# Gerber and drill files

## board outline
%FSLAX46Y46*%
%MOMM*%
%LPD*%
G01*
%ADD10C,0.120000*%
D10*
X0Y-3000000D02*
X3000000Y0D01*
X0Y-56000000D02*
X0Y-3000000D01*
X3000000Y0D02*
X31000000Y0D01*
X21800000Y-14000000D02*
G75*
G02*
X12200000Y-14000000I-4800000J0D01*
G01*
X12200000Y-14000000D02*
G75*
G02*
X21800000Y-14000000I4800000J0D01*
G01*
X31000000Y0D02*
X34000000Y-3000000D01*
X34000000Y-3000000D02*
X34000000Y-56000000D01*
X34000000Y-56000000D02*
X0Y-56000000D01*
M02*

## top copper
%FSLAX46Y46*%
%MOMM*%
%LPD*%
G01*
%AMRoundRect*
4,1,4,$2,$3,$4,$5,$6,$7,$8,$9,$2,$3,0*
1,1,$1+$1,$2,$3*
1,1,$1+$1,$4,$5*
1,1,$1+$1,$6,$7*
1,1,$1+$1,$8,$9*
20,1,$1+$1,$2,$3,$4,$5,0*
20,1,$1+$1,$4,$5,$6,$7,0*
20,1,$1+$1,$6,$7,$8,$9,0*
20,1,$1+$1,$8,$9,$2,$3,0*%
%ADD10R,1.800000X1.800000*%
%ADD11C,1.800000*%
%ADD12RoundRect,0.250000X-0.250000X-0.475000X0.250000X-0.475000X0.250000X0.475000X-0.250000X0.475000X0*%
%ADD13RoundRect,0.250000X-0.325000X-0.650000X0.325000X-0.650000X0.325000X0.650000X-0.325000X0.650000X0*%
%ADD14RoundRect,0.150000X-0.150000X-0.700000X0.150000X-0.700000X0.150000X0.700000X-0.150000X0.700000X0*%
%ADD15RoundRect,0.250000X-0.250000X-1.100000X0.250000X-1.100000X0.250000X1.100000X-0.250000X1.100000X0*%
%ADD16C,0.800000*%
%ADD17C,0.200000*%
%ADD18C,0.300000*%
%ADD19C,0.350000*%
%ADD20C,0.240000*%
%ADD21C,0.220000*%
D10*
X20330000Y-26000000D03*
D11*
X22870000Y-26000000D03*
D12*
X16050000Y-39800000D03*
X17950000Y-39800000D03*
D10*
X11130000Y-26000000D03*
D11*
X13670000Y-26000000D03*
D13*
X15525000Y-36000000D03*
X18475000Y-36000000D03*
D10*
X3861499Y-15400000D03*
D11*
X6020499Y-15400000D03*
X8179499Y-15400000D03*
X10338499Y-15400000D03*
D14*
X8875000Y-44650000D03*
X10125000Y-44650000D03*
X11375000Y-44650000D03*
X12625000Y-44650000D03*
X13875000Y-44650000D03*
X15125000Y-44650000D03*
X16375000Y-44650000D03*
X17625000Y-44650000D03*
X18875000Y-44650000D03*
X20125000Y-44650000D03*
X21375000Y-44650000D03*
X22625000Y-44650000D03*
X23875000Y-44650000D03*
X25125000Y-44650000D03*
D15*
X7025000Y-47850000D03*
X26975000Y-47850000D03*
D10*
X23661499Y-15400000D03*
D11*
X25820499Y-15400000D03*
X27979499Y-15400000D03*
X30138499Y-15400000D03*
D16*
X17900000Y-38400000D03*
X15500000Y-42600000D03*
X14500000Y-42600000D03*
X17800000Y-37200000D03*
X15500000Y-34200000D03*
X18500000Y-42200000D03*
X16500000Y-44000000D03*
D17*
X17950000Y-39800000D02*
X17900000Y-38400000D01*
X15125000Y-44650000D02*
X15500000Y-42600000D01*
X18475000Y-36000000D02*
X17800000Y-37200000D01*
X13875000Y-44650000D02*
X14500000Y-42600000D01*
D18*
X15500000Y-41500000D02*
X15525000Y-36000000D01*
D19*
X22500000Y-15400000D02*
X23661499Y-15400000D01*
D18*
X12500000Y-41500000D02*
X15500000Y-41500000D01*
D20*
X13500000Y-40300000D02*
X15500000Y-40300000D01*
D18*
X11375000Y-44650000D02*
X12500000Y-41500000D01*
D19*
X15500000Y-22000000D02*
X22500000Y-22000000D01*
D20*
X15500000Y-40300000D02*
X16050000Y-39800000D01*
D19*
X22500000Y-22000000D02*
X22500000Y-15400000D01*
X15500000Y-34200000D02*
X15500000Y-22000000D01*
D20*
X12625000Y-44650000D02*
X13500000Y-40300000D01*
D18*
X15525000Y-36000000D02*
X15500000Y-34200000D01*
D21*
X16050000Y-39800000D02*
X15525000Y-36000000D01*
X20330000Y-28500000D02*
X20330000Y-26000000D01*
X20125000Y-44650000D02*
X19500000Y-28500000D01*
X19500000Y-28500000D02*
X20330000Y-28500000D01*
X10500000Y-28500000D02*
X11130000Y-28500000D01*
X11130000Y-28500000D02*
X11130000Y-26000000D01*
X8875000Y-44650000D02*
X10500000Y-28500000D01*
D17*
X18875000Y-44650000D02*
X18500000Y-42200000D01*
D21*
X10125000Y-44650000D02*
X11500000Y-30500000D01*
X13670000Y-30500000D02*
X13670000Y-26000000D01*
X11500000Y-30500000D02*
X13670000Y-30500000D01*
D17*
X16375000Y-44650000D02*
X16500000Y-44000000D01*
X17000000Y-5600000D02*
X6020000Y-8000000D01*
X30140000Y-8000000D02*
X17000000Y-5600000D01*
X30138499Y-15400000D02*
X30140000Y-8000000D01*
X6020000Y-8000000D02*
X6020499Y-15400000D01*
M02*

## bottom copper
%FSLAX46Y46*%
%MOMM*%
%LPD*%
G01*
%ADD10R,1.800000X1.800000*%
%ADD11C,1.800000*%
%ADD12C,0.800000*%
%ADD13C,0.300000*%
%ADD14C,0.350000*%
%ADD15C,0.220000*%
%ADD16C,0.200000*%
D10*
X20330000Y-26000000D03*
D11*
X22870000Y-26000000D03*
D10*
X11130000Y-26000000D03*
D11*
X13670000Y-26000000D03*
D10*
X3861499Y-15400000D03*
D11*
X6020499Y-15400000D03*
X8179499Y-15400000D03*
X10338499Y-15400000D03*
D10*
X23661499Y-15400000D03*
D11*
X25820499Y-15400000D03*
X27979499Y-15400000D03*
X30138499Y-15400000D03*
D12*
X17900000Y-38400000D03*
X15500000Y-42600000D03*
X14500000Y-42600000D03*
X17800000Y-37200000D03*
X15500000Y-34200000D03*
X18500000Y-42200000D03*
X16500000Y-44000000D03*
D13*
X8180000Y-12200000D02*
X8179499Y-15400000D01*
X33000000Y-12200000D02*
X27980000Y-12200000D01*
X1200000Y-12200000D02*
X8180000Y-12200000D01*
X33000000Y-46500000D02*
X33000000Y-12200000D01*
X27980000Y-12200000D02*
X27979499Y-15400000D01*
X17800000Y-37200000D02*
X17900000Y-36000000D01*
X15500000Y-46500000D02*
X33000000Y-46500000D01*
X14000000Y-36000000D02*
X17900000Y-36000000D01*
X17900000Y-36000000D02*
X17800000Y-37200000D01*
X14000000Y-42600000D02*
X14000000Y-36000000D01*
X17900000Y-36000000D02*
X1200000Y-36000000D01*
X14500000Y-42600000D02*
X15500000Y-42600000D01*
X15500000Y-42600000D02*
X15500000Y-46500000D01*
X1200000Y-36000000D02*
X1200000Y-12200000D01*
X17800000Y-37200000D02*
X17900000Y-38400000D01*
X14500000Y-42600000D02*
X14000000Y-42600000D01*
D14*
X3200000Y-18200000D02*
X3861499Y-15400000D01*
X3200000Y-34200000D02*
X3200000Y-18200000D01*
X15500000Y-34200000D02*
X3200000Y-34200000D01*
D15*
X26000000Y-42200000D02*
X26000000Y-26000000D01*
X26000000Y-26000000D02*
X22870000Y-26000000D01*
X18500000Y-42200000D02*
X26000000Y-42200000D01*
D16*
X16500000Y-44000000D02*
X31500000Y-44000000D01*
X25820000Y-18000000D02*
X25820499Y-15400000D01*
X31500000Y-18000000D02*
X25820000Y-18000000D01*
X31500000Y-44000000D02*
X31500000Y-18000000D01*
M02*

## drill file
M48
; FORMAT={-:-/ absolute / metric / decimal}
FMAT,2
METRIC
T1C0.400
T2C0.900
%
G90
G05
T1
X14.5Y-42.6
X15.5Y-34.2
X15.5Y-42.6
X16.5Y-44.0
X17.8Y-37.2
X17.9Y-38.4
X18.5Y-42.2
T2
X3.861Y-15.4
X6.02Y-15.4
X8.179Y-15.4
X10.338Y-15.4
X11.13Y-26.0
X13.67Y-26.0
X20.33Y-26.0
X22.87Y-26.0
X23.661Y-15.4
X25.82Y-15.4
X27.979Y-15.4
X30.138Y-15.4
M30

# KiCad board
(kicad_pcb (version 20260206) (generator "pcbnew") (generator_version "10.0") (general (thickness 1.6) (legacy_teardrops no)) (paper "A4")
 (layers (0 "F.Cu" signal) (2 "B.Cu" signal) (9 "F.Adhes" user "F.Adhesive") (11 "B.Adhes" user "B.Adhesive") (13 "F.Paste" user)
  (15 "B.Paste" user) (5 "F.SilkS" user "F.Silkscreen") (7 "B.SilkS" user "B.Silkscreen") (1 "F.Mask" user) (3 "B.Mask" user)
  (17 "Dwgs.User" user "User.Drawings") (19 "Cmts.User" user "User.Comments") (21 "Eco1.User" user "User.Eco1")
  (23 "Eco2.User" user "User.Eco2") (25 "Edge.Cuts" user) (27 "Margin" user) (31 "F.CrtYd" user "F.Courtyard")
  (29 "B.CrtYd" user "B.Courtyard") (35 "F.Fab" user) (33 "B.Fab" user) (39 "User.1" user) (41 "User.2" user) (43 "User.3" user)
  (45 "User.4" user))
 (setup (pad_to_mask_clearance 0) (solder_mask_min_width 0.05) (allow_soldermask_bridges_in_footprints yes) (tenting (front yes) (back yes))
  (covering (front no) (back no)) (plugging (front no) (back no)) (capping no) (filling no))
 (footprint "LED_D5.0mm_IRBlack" (layer "F.Cu") (at 20.33 26)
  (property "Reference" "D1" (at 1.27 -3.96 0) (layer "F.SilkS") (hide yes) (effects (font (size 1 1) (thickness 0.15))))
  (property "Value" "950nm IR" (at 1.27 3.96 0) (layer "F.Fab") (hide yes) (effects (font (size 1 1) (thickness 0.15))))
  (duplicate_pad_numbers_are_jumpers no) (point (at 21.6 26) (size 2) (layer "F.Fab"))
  (pad "1" thru_hole rect (at 0 0) (size 1.8 1.8) (drill 0.9) (layers "*.Cu" "*.Mask") (remove_unused_layers no) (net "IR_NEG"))
  (pad "2" thru_hole circle (at 2.54 0) (size 1.8 1.8) (drill 0.9) (layers "*.Cu" "*.Mask") (remove_unused_layers no) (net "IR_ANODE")))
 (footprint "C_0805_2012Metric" (layer "F.Cu") (at 17 39.8)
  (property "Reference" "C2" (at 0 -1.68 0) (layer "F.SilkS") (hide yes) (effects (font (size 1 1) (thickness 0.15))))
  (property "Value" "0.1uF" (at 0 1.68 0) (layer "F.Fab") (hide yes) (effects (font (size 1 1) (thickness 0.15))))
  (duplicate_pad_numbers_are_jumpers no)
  (pad "1" smd roundrect (at -0.95 0) (size 1 1.45) (layers "F.Cu" "F.Mask" "F.Paste") (roundrect_rratio 0.25) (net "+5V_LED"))
  (pad "2" smd roundrect (at 0.95 0) (size 1 1.45) (layers "F.Cu" "F.Mask" "F.Paste") (roundrect_rratio 0.25) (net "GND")))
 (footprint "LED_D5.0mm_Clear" (layer "F.Cu") (at 11.13 26)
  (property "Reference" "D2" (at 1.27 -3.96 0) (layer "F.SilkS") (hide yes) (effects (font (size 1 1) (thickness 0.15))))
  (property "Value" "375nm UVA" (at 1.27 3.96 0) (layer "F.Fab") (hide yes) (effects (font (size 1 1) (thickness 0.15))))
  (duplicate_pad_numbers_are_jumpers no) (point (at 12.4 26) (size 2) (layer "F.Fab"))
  (pad "1" thru_hole rect (at 0 0) (size 1.8 1.8) (drill 0.9) (layers "*.Cu" "*.Mask") (remove_unused_layers no) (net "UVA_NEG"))
  (pad "2" thru_hole circle (at 2.54 0) (size 1.8 1.8) (drill 0.9) (layers "*.Cu" "*.Mask") (remove_unused_layers no) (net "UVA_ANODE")))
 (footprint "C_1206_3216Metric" (layer "F.Cu") (at 17 36)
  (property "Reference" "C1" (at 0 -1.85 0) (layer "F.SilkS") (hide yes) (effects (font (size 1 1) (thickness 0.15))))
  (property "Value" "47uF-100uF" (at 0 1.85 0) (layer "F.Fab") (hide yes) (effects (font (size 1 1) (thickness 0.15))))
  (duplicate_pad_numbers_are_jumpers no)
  (pad "1" smd roundrect (at -1.475 0) (size 1.15 1.8) (layers "F.Cu" "F.Mask" "F.Paste") (roundrect_rratio 0.217391) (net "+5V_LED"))
  (pad "2" smd roundrect (at 1.475 0) (size 1.15 1.8) (layers "F.Cu" "F.Mask" "F.Paste") (roundrect_rratio 0.217391) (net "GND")))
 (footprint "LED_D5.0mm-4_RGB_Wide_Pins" (layer "F.Cu") (at 3.861499 15.4)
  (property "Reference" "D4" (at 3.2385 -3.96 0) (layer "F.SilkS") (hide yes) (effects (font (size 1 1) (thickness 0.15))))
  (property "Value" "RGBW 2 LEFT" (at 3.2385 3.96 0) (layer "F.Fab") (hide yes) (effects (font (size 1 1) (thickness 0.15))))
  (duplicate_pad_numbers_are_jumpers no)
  (pad "1" thru_hole rect (at 0 0) (size 1.8 1.8) (drill 0.9) (layers "*.Cu" "*.Mask") (remove_unused_layers no) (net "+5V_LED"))
  (pad "2" thru_hole circle (at 2.159 0) (size 1.8 1.8) (drill 0.9) (layers "*.Cu" "*.Mask") (remove_unused_layers no) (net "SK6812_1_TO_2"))
  (pad "3" thru_hole circle (at 4.318 0) (size 1.8 1.8) (drill 0.9) (layers "*.Cu" "*.Mask") (remove_unused_layers no) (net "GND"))
  (pad "4" thru_hole circle (at 6.477 0) (size 1.8 1.8) (drill 0.9) (layers "*.Cu" "*.Mask") (remove_unused_layers no)))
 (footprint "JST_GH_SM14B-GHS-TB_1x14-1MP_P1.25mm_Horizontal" (layer "F.Cu") (at 17 46.5)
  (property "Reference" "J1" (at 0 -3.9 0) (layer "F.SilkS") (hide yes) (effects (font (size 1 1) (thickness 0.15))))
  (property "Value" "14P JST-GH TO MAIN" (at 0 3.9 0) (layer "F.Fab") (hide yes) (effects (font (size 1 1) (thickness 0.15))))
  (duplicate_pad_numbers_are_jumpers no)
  (pad "1" smd roundrect (at -8.125 -1.85) (size 0.6 1.7) (layers "F.Cu" "F.Mask" "F.Paste") (roundrect_rratio 0.25) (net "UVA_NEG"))
  (pad "2" smd roundrect (at -6.875 -1.85) (size 0.6 1.7) (layers "F.Cu" "F.Mask" "F.Paste") (roundrect_rratio 0.25) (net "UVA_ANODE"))
  (pad "3" smd roundrect (at -5.625 -1.85) (size 0.6 1.7) (layers "F.Cu" "F.Mask" "F.Paste") (roundrect_rratio 0.25) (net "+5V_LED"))
  (pad "4" smd roundrect (at -4.375 -1.85) (size 0.6 1.7) (layers "F.Cu" "F.Mask" "F.Paste") (roundrect_rratio 0.25) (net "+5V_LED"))
  (pad "5" smd roundrect (at -3.125 -1.85) (size 0.6 1.7) (layers "F.Cu" "F.Mask" "F.Paste") (roundrect_rratio 0.25) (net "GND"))
  (pad "6" smd roundrect (at -1.875 -1.85) (size 0.6 1.7) (layers "F.Cu" "F.Mask" "F.Paste") (roundrect_rratio 0.25) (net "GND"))
  (pad "7" smd roundrect (at -0.625 -1.85) (size 0.6 1.7) (layers "F.Cu" "F.Mask" "F.Paste") (roundrect_rratio 0.25) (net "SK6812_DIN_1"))
  (pad "8" smd roundrect (at 0.625 -1.85) (size 0.6 1.7) (layers "F.Cu" "F.Mask" "F.Paste") (roundrect_rratio 0.25))
  (pad "9" smd roundrect (at 1.875 -1.85) (size 0.6 1.7) (layers "F.Cu" "F.Mask" "F.Paste") (roundrect_rratio 0.25) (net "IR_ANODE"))
  (pad "10" smd roundrect (at 3.125 -1.85) (size 0.6 1.7) (layers "F.Cu" "F.Mask" "F.Paste") (roundrect_rratio 0.25) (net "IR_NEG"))
  (pad "11" smd roundrect (at 4.375 -1.85) (size 0.6 1.7) (layers "F.Cu" "F.Mask" "F.Paste") (roundrect_rratio 0.25))
  (pad "12" smd roundrect (at 5.625 -1.85) (size 0.6 1.7) (layers "F.Cu" "F.Mask" "F.Paste") (roundrect_rratio 0.25))
  (pad "13" smd roundrect (at 6.875 -1.85) (size 0.6 1.7) (layers "F.Cu" "F.Mask" "F.Paste") (roundrect_rratio 0.25))
  (pad "14" smd roundrect (at 8.125 -1.85) (size 0.6 1.7) (layers "F.Cu" "F.Mask" "F.Paste") (roundrect_rratio 0.25))
  (pad "MP" smd roundrect (at -9.975 1.35) (size 1 2.7) (layers "F.Cu" "F.Mask" "F.Paste") (roundrect_rratio 0.25))
  (pad "MP" smd roundrect (at 9.975 1.35) (size 1 2.7) (layers "F.Cu" "F.Mask" "F.Paste") (roundrect_rratio 0.25)))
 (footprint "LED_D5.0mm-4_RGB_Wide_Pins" (layer "F.Cu") (at 23.661499 15.4)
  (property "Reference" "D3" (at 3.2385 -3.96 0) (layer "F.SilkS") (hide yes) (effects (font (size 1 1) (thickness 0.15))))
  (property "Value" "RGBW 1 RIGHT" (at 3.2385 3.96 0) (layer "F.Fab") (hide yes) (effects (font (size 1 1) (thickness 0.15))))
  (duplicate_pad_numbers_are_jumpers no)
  (pad "1" thru_hole rect (at 0 0) (size 1.8 1.8) (drill 0.9) (layers "*.Cu" "*.Mask") (remove_unused_layers no) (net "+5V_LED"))
  (pad "2" thru_hole circle (at 2.159 0) (size 1.8 1.8) (drill 0.9) (layers "*.Cu" "*.Mask") (remove_unused_layers no) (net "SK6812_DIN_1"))
  (pad "3" thru_hole circle (at 4.318 0) (size 1.8 1.8) (drill 0.9) (layers "*.Cu" "*.Mask") (remove_unused_layers no) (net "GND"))
  (pad "4" thru_hole circle (at 6.477 0) (size 1.8 1.8) (drill 0.9) (layers "*.Cu" "*.Mask") (remove_unused_layers no) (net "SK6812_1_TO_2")))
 (gr_line (start 0 3) (end 3 0) (stroke (width 0.12) (type default)) (layer "Edge.Cuts"))
 (gr_line (start 0 56) (end 0 3) (stroke (width 0.12) (type default)) (layer "Edge.Cuts"))
 (gr_line (start 3 0) (end 31 0) (stroke (width 0.12) (type default)) (layer "Edge.Cuts"))
 (gr_circle (center 17 14) (end 21.8 14) (stroke (width 0.12) (type default)) (fill no) (layer "Edge.Cuts"))
 (gr_line (start 31 0) (end 34 3) (stroke (width 0.12) (type default)) (layer "Edge.Cuts"))
 (gr_line (start 34 3) (end 34 56) (stroke (width 0.12) (type default)) (layer "Edge.Cuts"))
 (gr_line (start 34 56) (end 0 56) (stroke (width 0.12) (type default)) (layer "Edge.Cuts"))
 (segment (start 17.95 39.8) (end 17.9 38.4) (width 0.2) (layer "F.Cu") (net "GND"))
 (segment (start 15.125 44.65) (end 15.5 42.6) (width 0.2) (layer "F.Cu") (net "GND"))
 (segment (start 18.475 36) (end 17.8 37.2) (width 0.2) (layer "F.Cu") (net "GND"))
 (segment (start 13.875 44.65) (end 14.5 42.6) (width 0.2) (layer "F.Cu") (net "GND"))
 (via (at 17.9 38.4) (size 0.8) (drill 0.4) (layers "F.Cu" "B.Cu") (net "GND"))
 (via (at 15.5 42.6) (size 0.8) (drill 0.4) (layers "F.Cu" "B.Cu") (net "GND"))
 (via (at 14.5 42.6) (size 0.8) (drill 0.4) (layers "F.Cu" "B.Cu") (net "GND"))
 (via (at 17.8 37.2) (size 0.8) (drill 0.4) (layers "F.Cu" "B.Cu") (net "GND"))
 (segment (start 8.18 12.2) (end 8.179499 15.4) (width 0.3) (layer "B.Cu") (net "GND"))
 (segment (start 33 12.2) (end 27.98 12.2) (width 0.3) (layer "B.Cu") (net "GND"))
 (segment (start 1.2 12.2) (end 8.18 12.2) (width 0.3) (layer "B.Cu") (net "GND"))
 (segment (start 33 46.5) (end 33 12.2) (width 0.3) (layer "B.Cu") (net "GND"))
 (segment (start 27.98 12.2) (end 27.979499 15.4) (width 0.3) (layer "B.Cu") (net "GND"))
 (segment (start 17.8 37.2) (end 17.9 36) (width 0.3) (layer "B.Cu") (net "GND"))
 (segment (start 15.5 46.5) (end 33 46.5) (width 0.3) (layer "B.Cu") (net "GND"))
 (segment (start 14 36) (end 17.9 36) (width 0.3) (layer "B.Cu") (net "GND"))
 (segment (start 17.9 36) (end 17.8 37.2) (width 0.3) (layer "B.Cu") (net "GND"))
 (segment (start 14 42.6) (end 14 36) (width 0.3) (layer "B.Cu") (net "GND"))
 (segment (start 17.9 36) (end 1.2 36) (width 0.3) (layer "B.Cu") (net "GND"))
 (segment (start 14.5 42.6) (end 15.5 42.6) (width 0.3) (layer "B.Cu") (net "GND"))
 (segment (start 15.5 42.6) (end 15.5 46.5) (width 0.3) (layer "B.Cu") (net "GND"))
 (segment (start 1.2 36) (end 1.2 12.2) (width 0.3) (layer "B.Cu") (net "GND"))
 (segment (start 17.8 37.2) (end 17.9 38.4) (width 0.3) (layer "B.Cu") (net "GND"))
 (segment (start 14.5 42.6) (end 14 42.6) (width 0.3) (layer "B.Cu") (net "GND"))
 (segment (start 15.5 41.5) (end 15.525 36) (width 0.3) (layer "F.Cu") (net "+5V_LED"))
 (segment (start 22.5 15.4) (end 23.661499 15.4) (width 0.35) (layer "F.Cu") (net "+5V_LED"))
 (segment (start 12.5 41.5) (end 15.5 41.5) (width 0.3) (layer "F.Cu") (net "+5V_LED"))
 (segment (start 13.5 40.3) (end 15.5 40.3) (width 0.24) (layer "F.Cu") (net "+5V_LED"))
 (segment (start 11.375 44.65) (end 12.5 41.5) (width 0.3) (layer "F.Cu") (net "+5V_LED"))
 (segment (start 15.5 22) (end 22.5 22) (width 0.35) (layer "F.Cu") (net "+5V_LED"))
 (segment (start 15.5 40.3) (end 16.05 39.8) (width 0.24) (layer "F.Cu") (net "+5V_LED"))
 (segment (start 22.5 22) (end 22.5 15.4) (width 0.35) (layer "F.Cu") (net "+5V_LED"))
 (segment (start 15.5 34.2) (end 15.5 22) (width 0.35) (layer "F.Cu") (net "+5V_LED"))
 (segment (start 12.625 44.65) (end 13.5 40.3) (width 0.24) (layer "F.Cu") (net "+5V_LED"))
 (segment (start 15.525 36) (end 15.5 34.2) (width 0.3) (layer "F.Cu") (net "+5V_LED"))
 (segment (start 16.05 39.8) (end 15.525 36) (width 0.22) (layer "F.Cu") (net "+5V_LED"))
 (via (at 15.5 34.2) (size 0.8) (drill 0.4) (layers "F.Cu" "B.Cu") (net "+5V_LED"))
 (segment (start 3.2 18.2) (end 3.861499 15.4) (width 0.35) (layer "B.Cu") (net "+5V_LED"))
 (segment (start 3.2 34.2) (end 3.2 18.2) (width 0.35) (layer "B.Cu") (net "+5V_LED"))
 (segment (start 15.5 34.2) (end 3.2 34.2) (width 0.35) (layer "B.Cu") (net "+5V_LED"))
 (segment (start 20.33 28.5) (end 20.33 26) (width 0.22) (layer "F.Cu") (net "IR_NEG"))
 (segment (start 20.125 44.65) (end 19.5 28.5) (width 0.22) (layer "F.Cu") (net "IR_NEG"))
 (segment (start 19.5 28.5) (end 20.33 28.5) (width 0.22) (layer "F.Cu") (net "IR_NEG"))
 (segment (start 10.5 28.5) (end 11.13 28.5) (width 0.22) (layer "F.Cu") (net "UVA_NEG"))
 (segment (start 11.13 28.5) (end 11.13 26) (width 0.22) (layer "F.Cu") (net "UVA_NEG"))
 (segment (start 8.875 44.65) (end 10.5 28.5) (width 0.22) (layer "F.Cu") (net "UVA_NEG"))
 (segment (start 18.875 44.65) (end 18.5 42.2) (width 0.2) (layer "F.Cu") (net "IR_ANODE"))
 (via (at 18.5 42.2) (size 0.8) (drill 0.4) (layers "F.Cu" "B.Cu") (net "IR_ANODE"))
 (segment (start 26 42.2) (end 26 26) (width 0.22) (layer "B.Cu") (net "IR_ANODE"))
 (segment (start 26 26) (end 22.87 26) (width 0.22) (layer "B.Cu") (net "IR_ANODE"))
 (segment (start 18.5 42.2) (end 26 42.2) (width 0.22) (layer "B.Cu") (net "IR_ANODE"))
 (segment (start 10.125 44.65) (end 11.5 30.5) (width 0.22) (layer "F.Cu") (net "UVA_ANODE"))
 (segment (start 13.67 30.5) (end 13.67 26) (width 0.22) (layer "F.Cu") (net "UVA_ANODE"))
 (segment (start 11.5 30.5) (end 13.67 30.5) (width 0.22) (layer "F.Cu") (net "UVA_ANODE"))
 (segment (start 16.375 44.65) (end 16.5 44) (width 0.2) (layer "F.Cu") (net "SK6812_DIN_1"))
 (via (at 16.5 44) (size 0.8) (drill 0.4) (layers "F.Cu" "B.Cu") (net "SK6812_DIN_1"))
 (segment (start 16.5 44) (end 31.5 44) (width 0.2) (layer "B.Cu") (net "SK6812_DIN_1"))
 (segment (start 25.82 18) (end 25.820499 15.4) (width 0.2) (layer "B.Cu") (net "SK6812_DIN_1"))
 (segment (start 31.5 18) (end 25.82 18) (width 0.2) (layer "B.Cu") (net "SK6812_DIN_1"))
 (segment (start 31.5 44) (end 31.5 18) (width 0.2) (layer "B.Cu") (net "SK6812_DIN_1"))
 (segment (start 17 5.6) (end 6.02 8) (width 0.2) (layer "F.Cu") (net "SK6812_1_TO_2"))
 (segment (start 30.14 8) (end 17 5.6) (width 0.2) (layer "F.Cu") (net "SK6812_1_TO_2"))
 (segment (start 30.138499 15.4) (end 30.14 8) (width 0.2) (layer "F.Cu") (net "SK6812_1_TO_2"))
 (segment (start 6.02 8) (end 6.020499 15.4) (width 0.2) (layer "F.Cu") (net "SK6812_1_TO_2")))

